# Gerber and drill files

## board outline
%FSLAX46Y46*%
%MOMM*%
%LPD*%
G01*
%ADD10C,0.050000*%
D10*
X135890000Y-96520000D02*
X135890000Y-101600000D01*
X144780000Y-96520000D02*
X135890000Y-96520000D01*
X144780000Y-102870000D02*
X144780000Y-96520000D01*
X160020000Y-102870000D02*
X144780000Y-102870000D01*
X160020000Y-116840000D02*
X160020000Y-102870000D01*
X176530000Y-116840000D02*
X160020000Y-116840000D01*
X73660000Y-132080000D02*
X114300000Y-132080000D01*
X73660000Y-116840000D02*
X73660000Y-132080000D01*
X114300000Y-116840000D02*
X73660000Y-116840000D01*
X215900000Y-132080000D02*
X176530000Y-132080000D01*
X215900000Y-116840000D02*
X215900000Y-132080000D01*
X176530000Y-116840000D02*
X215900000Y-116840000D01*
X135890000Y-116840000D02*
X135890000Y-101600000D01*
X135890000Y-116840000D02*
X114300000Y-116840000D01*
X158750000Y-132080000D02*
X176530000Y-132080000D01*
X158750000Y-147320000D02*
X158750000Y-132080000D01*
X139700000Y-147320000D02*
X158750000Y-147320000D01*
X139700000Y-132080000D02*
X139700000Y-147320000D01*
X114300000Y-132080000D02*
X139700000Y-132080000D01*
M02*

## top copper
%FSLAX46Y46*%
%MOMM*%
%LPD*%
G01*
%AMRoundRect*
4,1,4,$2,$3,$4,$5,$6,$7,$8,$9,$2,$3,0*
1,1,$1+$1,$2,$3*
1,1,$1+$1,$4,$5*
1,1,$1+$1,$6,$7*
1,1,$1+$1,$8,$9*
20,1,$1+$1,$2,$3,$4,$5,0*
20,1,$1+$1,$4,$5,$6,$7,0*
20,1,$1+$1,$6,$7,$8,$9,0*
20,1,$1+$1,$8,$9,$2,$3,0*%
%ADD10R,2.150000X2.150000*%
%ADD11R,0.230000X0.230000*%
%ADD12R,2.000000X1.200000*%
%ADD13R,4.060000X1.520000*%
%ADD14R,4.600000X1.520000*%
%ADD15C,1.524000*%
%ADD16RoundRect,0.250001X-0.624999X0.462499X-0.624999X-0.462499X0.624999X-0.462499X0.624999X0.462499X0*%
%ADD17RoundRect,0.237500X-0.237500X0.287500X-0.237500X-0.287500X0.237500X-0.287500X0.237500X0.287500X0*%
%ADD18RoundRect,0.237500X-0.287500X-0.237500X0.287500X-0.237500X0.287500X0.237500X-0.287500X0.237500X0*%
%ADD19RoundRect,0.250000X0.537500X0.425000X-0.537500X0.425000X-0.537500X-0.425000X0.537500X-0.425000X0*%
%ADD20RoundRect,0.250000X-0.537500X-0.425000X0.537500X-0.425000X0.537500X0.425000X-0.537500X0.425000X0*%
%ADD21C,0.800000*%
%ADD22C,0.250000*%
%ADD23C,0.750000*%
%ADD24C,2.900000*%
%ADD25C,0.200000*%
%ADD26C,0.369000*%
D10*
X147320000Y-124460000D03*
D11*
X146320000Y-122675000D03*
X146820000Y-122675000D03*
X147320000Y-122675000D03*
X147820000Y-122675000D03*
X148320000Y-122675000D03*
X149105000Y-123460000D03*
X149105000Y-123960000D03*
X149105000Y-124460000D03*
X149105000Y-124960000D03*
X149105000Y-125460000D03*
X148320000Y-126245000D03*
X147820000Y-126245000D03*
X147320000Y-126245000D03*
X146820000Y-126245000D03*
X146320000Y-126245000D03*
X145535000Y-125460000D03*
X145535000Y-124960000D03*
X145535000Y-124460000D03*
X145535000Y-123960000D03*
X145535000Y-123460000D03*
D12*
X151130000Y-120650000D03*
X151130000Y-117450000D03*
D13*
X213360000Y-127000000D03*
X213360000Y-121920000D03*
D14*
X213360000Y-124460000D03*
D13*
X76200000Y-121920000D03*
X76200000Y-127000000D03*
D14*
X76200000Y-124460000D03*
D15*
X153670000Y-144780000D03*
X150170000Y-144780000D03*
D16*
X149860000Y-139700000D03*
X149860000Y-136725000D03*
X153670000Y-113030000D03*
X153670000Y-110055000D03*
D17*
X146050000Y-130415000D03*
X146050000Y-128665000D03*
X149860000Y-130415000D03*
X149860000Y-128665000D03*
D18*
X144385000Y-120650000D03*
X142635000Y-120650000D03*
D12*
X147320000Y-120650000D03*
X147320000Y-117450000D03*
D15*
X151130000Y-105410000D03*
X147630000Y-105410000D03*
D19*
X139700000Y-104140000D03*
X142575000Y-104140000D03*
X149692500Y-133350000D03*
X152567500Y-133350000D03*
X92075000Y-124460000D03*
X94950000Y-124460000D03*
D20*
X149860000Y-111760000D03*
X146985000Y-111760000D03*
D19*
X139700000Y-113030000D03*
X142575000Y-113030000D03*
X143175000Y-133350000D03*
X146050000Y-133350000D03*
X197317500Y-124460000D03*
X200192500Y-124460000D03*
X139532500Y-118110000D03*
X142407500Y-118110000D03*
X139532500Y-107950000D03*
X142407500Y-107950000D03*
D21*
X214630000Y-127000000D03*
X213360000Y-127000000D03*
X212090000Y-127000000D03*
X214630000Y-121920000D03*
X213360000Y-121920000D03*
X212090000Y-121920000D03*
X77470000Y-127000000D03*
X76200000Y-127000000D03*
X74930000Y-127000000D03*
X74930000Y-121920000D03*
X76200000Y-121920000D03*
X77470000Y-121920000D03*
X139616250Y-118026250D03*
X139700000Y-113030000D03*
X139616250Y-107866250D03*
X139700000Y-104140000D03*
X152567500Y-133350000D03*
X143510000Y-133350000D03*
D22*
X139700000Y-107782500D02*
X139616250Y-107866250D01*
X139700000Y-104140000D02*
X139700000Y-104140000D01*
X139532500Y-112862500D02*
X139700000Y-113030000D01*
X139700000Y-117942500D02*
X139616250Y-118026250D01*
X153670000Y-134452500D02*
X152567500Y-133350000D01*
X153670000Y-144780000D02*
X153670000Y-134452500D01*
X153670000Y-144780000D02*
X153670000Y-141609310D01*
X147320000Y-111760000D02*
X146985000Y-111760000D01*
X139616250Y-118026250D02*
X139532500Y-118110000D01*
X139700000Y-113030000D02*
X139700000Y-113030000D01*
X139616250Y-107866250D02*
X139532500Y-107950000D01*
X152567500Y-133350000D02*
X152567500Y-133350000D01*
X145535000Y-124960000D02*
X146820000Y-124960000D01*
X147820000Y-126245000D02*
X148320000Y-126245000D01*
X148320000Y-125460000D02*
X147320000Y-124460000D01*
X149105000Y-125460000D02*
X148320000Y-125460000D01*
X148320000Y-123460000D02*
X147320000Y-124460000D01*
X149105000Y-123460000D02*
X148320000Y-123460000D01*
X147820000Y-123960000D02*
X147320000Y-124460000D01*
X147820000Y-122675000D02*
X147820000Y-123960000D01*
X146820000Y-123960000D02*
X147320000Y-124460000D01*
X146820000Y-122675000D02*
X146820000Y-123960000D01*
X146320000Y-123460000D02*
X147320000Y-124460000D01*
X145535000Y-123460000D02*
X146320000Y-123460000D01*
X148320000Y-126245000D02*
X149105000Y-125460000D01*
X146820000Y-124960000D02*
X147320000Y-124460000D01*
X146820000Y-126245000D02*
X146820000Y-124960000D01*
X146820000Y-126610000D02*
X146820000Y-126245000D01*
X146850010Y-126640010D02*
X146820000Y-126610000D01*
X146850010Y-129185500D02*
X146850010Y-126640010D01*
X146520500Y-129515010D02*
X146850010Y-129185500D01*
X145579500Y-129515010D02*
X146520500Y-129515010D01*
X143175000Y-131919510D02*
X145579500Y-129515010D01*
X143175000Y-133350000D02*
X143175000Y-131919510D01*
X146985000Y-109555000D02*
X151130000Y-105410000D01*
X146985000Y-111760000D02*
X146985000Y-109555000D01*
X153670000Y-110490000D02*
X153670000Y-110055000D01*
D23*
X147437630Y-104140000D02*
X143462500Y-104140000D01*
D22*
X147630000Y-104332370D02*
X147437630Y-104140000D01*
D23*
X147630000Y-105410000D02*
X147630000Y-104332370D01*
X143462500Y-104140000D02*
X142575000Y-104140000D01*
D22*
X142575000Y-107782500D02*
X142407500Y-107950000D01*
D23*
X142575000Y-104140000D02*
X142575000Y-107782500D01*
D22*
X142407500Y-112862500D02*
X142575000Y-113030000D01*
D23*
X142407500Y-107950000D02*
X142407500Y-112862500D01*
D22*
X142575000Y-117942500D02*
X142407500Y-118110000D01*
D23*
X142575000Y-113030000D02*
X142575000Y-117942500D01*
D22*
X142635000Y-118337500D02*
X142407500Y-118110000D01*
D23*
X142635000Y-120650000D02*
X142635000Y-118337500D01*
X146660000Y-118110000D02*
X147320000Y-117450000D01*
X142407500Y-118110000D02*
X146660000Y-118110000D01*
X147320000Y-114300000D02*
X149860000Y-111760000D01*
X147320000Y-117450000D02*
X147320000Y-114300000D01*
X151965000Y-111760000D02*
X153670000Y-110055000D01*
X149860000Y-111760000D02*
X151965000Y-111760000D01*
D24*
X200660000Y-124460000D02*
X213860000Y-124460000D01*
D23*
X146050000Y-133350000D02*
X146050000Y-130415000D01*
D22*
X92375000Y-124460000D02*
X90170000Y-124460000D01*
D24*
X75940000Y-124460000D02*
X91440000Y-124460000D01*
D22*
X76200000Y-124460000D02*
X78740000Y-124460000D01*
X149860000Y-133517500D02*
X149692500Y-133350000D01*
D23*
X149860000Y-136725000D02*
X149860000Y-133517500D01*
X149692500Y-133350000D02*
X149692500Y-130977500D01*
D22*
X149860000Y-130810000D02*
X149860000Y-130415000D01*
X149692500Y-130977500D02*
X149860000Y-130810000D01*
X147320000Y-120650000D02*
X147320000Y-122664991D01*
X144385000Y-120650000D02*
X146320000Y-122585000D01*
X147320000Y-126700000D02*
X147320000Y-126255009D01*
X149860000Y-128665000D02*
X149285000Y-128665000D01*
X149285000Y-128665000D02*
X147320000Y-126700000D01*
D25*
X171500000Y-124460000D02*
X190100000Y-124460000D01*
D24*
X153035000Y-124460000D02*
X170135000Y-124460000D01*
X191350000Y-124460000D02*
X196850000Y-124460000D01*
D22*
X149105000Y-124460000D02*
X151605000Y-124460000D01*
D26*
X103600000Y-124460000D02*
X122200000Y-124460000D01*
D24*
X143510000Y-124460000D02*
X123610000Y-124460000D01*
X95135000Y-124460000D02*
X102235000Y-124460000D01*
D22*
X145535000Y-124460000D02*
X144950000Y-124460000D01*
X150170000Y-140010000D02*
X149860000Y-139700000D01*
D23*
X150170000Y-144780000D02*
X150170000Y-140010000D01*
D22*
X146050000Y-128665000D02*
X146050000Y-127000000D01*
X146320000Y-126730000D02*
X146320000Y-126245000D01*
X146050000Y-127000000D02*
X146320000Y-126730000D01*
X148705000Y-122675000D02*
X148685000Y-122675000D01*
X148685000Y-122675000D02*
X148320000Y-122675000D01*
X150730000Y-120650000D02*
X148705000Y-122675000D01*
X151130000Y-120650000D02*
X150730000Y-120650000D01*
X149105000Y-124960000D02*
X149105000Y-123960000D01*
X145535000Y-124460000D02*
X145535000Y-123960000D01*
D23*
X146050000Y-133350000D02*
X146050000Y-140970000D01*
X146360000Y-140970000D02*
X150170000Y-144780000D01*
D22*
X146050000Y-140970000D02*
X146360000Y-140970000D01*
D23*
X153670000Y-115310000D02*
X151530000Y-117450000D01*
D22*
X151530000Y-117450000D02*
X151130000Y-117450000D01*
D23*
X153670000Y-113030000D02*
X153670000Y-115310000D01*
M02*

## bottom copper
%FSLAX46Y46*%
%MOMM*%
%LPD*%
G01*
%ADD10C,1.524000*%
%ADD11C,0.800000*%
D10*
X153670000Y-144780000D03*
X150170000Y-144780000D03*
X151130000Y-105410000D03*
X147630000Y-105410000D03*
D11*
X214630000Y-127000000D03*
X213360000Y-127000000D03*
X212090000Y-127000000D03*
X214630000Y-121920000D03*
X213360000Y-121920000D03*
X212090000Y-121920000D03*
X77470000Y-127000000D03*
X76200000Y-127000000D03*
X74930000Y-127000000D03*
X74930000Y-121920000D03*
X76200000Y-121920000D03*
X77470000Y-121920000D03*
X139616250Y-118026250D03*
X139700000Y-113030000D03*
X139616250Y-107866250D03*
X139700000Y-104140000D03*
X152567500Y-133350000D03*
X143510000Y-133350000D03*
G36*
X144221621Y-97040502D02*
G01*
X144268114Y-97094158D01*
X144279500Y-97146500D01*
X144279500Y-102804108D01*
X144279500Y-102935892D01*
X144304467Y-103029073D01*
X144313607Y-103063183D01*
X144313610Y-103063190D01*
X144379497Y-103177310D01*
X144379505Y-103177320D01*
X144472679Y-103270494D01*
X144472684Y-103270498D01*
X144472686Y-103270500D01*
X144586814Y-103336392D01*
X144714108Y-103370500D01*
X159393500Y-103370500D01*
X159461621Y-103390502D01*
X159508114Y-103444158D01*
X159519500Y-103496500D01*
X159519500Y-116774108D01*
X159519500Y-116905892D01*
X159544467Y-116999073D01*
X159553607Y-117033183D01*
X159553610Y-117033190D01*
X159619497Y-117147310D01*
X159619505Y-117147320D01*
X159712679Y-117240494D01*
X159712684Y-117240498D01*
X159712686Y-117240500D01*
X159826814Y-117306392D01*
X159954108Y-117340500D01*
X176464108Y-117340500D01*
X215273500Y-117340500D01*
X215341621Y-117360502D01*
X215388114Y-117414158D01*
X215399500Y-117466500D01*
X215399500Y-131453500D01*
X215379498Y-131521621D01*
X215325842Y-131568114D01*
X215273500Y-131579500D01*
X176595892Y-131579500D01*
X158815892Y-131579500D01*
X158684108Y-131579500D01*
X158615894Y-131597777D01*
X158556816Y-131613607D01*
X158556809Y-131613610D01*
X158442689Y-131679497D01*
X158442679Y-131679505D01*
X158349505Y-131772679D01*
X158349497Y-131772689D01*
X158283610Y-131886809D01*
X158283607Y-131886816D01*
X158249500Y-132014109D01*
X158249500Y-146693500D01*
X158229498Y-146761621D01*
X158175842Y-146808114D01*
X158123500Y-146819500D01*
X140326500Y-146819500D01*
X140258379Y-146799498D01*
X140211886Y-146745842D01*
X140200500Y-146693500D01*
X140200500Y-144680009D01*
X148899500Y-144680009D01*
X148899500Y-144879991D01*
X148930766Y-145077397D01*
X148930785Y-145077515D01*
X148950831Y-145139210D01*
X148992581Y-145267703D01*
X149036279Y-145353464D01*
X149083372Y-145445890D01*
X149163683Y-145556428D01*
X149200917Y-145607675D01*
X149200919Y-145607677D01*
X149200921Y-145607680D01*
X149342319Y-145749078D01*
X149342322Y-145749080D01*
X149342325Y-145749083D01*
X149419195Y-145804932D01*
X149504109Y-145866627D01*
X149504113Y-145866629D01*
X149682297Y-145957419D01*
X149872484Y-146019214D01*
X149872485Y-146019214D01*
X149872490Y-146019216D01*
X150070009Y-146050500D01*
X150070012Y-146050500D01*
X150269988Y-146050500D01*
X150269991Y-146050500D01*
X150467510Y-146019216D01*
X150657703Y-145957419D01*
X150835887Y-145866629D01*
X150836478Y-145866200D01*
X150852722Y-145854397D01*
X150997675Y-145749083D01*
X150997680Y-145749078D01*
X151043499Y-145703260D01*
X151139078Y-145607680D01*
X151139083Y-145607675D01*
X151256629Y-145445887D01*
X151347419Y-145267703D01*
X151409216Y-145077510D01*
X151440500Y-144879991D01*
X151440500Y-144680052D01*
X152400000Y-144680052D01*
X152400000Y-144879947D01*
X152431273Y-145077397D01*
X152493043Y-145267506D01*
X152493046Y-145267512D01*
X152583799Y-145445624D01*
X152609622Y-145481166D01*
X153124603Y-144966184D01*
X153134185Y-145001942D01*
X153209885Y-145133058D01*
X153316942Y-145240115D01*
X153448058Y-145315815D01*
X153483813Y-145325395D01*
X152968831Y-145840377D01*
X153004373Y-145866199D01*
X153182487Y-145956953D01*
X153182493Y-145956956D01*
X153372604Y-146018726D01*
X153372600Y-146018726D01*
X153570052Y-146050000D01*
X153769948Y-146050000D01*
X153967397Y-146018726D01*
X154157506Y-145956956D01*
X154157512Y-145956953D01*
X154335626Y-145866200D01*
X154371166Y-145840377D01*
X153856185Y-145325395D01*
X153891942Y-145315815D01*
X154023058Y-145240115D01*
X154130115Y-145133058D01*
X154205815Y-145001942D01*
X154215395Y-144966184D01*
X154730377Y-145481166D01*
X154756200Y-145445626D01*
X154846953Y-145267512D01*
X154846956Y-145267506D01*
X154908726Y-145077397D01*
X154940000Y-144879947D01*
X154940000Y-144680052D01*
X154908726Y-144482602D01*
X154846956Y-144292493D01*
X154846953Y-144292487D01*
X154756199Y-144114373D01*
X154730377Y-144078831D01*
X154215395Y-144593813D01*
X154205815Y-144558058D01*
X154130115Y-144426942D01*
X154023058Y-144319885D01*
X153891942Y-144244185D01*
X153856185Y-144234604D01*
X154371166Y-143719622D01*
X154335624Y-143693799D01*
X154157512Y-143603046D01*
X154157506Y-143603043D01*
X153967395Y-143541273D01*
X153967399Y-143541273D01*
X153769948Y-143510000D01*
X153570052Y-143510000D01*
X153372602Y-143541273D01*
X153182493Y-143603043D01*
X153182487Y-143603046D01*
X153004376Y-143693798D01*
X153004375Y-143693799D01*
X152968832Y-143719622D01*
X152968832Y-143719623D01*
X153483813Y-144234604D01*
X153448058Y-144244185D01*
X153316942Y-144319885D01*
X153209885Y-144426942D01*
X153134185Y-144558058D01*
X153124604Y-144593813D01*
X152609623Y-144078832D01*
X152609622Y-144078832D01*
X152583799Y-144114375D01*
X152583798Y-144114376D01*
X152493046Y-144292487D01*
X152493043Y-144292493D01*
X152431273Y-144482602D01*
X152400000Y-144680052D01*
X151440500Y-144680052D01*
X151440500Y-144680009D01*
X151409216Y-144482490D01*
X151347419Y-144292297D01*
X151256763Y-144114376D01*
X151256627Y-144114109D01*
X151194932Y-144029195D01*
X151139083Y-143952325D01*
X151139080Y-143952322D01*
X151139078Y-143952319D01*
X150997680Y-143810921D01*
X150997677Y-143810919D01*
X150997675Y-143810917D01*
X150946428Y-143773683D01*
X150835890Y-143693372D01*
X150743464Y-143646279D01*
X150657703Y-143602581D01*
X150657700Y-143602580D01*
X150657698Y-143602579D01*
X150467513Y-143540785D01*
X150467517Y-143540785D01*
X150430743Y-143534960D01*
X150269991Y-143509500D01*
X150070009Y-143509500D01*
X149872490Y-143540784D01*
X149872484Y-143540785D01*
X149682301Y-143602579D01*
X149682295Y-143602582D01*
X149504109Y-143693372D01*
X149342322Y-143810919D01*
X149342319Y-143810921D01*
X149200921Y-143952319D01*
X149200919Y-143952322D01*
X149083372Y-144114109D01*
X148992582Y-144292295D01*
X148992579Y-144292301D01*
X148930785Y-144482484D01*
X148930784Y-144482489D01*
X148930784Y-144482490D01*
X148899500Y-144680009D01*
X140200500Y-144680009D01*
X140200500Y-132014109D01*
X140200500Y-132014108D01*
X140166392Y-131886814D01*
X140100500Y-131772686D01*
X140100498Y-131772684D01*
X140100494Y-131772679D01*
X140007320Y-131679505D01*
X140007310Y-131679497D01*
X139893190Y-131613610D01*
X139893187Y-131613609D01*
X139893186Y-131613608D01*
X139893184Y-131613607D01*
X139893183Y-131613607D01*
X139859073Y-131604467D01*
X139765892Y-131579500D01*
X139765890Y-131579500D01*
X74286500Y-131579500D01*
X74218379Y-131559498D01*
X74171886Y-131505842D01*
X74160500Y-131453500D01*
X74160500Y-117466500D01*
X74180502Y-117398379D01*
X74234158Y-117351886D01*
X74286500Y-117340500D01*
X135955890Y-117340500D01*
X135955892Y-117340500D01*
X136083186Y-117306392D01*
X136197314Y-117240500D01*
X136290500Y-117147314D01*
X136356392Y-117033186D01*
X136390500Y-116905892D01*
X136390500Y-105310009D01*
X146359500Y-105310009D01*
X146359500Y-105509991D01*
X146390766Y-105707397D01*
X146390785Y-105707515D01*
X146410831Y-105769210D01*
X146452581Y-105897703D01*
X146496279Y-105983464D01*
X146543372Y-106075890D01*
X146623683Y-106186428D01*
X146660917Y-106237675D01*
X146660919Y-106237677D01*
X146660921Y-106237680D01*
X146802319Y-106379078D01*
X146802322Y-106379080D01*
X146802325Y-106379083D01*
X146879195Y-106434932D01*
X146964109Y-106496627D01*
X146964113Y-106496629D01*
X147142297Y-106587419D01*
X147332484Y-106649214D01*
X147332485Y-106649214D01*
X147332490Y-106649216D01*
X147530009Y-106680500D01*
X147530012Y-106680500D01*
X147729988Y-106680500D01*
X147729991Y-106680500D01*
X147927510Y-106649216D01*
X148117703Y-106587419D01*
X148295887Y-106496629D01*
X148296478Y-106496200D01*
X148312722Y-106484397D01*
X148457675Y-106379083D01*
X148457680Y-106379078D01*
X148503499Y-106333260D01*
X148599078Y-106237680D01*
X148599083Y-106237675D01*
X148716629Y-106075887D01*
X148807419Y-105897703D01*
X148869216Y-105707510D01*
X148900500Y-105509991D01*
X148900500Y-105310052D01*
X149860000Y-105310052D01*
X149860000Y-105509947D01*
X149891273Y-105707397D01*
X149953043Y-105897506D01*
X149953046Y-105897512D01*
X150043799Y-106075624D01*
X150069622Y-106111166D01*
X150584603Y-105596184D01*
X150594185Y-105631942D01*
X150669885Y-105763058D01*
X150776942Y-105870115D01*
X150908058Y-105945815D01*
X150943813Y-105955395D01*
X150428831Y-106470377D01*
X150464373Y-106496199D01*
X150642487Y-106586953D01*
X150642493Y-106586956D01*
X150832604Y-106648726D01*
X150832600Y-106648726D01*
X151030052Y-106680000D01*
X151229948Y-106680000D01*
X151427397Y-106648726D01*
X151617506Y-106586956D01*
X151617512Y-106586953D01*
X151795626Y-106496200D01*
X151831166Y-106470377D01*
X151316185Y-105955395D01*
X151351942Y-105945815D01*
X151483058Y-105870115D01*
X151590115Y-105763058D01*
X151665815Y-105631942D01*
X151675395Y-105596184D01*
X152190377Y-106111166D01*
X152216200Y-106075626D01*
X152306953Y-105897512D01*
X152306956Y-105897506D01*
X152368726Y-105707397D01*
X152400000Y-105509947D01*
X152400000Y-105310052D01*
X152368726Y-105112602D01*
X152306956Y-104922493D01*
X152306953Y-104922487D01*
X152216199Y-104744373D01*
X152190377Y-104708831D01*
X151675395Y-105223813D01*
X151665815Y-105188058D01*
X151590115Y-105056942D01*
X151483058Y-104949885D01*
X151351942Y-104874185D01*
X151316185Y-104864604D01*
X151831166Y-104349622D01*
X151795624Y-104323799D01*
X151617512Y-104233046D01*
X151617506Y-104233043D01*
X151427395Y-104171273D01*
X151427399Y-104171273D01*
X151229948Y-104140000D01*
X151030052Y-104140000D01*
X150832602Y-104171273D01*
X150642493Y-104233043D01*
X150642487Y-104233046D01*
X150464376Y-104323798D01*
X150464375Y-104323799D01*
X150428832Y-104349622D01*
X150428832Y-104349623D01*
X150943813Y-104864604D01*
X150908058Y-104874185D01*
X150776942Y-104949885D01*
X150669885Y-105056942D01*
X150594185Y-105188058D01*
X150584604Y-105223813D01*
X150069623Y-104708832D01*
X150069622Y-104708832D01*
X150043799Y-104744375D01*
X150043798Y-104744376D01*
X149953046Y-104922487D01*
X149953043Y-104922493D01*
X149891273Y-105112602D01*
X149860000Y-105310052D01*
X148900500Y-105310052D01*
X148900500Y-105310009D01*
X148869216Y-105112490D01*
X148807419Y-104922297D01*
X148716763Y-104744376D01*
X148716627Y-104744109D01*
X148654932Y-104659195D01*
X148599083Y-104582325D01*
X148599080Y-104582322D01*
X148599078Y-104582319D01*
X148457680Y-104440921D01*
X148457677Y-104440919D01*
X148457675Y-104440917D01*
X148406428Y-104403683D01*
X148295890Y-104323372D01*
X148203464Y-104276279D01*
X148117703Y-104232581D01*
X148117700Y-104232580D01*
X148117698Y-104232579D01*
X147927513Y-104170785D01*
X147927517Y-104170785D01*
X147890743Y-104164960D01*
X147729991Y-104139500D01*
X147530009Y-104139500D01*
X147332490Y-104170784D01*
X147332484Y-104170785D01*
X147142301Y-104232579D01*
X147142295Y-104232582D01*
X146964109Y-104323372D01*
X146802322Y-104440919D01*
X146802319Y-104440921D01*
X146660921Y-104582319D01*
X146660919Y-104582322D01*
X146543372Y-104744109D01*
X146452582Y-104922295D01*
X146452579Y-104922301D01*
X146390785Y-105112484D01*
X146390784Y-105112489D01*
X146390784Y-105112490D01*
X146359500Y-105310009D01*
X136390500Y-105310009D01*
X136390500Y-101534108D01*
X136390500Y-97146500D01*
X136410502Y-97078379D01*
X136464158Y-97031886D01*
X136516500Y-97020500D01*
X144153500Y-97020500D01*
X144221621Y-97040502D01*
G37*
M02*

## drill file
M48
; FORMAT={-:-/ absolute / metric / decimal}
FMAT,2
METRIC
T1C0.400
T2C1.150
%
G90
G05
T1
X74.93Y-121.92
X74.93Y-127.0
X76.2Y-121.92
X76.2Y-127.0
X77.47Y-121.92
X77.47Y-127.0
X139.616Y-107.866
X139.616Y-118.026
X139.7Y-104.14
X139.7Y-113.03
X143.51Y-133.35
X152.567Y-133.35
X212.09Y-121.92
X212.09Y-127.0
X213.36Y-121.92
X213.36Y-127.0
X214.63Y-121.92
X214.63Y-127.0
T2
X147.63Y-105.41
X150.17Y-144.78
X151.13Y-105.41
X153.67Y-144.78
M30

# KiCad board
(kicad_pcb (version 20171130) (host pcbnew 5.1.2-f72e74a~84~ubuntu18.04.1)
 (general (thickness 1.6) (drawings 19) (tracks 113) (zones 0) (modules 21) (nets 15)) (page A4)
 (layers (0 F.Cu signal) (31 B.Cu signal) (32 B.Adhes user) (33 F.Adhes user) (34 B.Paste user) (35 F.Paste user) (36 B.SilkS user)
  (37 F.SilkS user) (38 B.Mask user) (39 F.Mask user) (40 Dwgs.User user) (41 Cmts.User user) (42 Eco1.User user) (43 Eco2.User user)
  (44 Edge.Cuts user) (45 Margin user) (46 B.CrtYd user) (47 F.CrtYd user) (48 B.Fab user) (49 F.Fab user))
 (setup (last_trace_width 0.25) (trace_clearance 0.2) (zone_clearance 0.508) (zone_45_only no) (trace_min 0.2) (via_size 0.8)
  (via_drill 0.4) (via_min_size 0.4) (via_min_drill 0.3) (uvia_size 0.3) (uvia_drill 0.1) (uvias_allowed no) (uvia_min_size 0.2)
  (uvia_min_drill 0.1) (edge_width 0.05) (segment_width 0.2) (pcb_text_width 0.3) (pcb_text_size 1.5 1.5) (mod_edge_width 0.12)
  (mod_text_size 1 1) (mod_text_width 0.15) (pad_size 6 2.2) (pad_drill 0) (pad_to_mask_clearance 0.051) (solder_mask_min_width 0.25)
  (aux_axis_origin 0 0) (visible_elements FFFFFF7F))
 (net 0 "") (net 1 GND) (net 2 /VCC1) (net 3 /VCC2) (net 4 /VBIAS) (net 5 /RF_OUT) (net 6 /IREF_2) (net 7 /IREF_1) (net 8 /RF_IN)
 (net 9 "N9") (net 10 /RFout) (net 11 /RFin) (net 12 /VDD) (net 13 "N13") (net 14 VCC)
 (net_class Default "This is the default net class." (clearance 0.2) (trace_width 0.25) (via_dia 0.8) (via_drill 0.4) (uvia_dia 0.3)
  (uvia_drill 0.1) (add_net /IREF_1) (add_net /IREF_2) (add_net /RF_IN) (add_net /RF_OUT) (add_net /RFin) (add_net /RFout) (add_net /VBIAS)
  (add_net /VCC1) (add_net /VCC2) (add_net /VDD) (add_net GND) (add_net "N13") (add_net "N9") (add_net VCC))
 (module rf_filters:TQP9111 (layer F.Cu) (at 147.32 124.46)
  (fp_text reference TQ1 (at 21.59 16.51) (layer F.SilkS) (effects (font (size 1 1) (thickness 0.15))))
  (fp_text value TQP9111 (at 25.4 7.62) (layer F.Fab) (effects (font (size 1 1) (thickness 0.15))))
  (pad 21 smd rect (at 0 0) (size 2.15 2.15) (layers F.Cu F.Paste F.Mask) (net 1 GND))
  (pad 20 smd rect (at -1 -1.785) (size 0.23 0.23) (layers F.Cu F.Paste F.Mask) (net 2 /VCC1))
  (pad 19 smd rect (at -0.5 -1.785) (size 0.23 0.23) (layers F.Cu F.Paste F.Mask) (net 1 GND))
  (pad 18 smd rect (at 0 -1.785) (size 0.23 0.23) (layers F.Cu F.Paste F.Mask) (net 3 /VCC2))
  (pad 17 smd rect (at 0.5 -1.785) (size 0.23 0.23) (layers F.Cu F.Paste F.Mask) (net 1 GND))
  (pad 16 smd rect (at 1 -1.785) (size 0.23 0.23) (layers F.Cu F.Paste F.Mask) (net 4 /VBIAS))
  (pad 15 smd rect (at 1.785 -1) (size 0.23 0.23) (layers F.Cu F.Paste F.Mask) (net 1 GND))
  (pad 14 smd rect (at 1.785 -0.5) (size 0.23 0.23) (layers F.Cu F.Paste F.Mask) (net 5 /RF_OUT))
  (pad 13 smd rect (at 1.785 0) (size 0.23 0.23) (layers F.Cu F.Paste F.Mask) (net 5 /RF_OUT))
  (pad 12 smd rect (at 1.785 0.5) (size 0.23 0.23) (layers F.Cu F.Paste F.Mask) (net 5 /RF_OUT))
  (pad 11 smd rect (at 1.785 1) (size 0.23 0.23) (layers F.Cu F.Paste F.Mask) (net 1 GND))
  (pad 10 smd rect (at 1 1.785) (size 0.23 0.23) (layers F.Cu F.Paste F.Mask) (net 1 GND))
  (pad 9 smd rect (at 0.5 1.785) (size 0.23 0.23) (layers F.Cu F.Paste F.Mask) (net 1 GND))
  (pad 8 smd rect (at 0 1.785) (size 0.23 0.23) (layers F.Cu F.Paste F.Mask) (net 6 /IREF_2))
  (pad 7 smd rect (at -0.5 1.785) (size 0.23 0.23) (layers F.Cu F.Paste F.Mask) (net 1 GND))
  (pad 6 smd rect (at -1 1.785) (size 0.23 0.23) (layers F.Cu F.Paste F.Mask) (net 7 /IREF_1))
  (pad 5 smd rect (at -1.785 1) (size 0.23 0.23) (layers F.Cu F.Paste F.Mask))
  (pad 4 smd rect (at -1.785 0.5) (size 0.23 0.23) (layers F.Cu F.Paste F.Mask) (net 1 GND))
  (pad 3 smd rect (at -1.785 0) (size 0.23 0.23) (layers F.Cu F.Paste F.Mask) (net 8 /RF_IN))
  (pad 2 smd rect (at -1.785 -0.5) (size 0.23 0.23) (layers F.Cu F.Paste F.Mask) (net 8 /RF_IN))
  (pad 1 smd rect (at -1.785 -1) (size 0.23 0.23) (layers F.Cu F.Paste F.Mask) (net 1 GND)))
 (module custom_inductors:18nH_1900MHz (layer F.Cu) (at 151.13 119.05)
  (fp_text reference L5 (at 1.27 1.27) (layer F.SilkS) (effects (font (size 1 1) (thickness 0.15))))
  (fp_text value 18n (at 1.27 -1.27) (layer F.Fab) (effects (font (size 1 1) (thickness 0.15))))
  (pad 2 smd rect (at 0 1.6) (size 2 1.2) (layers F.Cu F.Paste F.Mask) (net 4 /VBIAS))
  (pad 1 smd rect (at 0 -1.6) (size 2 1.2) (layers F.Cu F.Paste F.Mask) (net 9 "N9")))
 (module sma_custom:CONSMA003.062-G (layer F.Cu) (at 217.17 127)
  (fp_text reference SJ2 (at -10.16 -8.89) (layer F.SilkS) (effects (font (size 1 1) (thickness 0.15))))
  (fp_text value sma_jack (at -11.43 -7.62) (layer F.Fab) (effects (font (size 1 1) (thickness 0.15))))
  (pad 3 smd rect (at -3.81 0) (size 4.06 1.52) (layers F.Cu F.Paste F.Mask) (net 1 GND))
  (pad 2 smd rect (at -3.81 -5.08) (size 4.06 1.52) (layers F.Cu F.Paste F.Mask) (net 1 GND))
  (pad 1 smd rect (at -3.81 -2.54) (size 4.6 1.52) (layers F.Cu F.Paste F.Mask) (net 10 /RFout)))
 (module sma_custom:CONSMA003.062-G (layer F.Cu) (at 72.39 121.92 180)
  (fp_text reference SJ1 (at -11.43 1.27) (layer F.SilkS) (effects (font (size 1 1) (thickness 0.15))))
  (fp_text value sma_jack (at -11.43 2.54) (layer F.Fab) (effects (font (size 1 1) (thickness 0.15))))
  (pad 3 smd rect (at -3.81 0 180) (size 4.06 1.52) (layers F.Cu F.Paste F.Mask) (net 1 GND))
  (pad 2 smd rect (at -3.81 -5.08 180) (size 4.06 1.52) (layers F.Cu F.Paste F.Mask) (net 1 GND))
  (pad 1 smd rect (at -3.81 -2.54 180) (size 4.6 1.52) (layers F.Cu F.Paste F.Mask) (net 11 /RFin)))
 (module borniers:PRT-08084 (layer F.Cu) (at 153.67 149.86)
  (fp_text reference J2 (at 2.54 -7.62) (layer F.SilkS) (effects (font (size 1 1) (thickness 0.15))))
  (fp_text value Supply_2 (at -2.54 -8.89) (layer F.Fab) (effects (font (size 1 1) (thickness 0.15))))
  (pad 2 thru_hole circle (at 0 -5.08) (size 1.524 1.524) (drill 1.15) (layers *.Cu *.Mask) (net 1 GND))
  (pad 1 thru_hole circle (at -3.5 -5.08) (size 1.524 1.524) (drill 1.15) (layers *.Cu *.Mask) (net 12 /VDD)))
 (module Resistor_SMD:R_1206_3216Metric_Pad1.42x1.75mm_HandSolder (layer F.Cu) (at 149.86 138.2125 270)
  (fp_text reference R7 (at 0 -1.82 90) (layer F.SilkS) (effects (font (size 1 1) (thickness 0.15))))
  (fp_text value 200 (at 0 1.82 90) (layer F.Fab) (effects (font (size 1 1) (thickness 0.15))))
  (pad 2 smd roundrect (at 1.4875 0 270) (size 1.425 1.75) (layers F.Cu F.Paste F.Mask) (roundrect_rratio 0.175439) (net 12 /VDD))
  (pad 1 smd roundrect (at -1.4875 0 270) (size 1.425 1.75) (layers F.Cu F.Paste F.Mask) (roundrect_rratio 0.175439) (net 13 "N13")))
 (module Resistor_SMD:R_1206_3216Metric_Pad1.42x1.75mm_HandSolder (layer F.Cu) (at 153.67 111.5425 270)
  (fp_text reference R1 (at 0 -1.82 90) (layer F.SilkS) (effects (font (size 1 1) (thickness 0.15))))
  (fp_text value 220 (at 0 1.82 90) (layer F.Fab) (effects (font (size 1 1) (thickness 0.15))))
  (pad 2 smd roundrect (at 1.4875 0 270) (size 1.425 1.75) (layers F.Cu F.Paste F.Mask) (roundrect_rratio 0.175439) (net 9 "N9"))
  (pad 1 smd roundrect (at -1.4875 0 270) (size 1.425 1.75) (layers F.Cu F.Paste F.Mask) (roundrect_rratio 0.175439) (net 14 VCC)))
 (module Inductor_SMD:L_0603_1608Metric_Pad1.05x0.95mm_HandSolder (layer F.Cu) (at 146.05 129.54 270)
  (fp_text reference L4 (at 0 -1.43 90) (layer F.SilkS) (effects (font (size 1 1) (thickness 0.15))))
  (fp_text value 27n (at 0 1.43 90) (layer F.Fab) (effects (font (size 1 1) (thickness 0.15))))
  (pad 2 smd roundrect (at 0.875 0 270) (size 1.05 0.95) (layers F.Cu F.Paste F.Mask) (roundrect_rratio 0.25) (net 12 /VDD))
  (pad 1 smd roundrect (at -0.875 0 270) (size 1.05 0.95) (layers F.Cu F.Paste F.Mask) (roundrect_rratio 0.25) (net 7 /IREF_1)))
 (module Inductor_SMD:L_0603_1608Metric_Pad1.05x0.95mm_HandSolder (layer F.Cu) (at 149.86 129.54 270)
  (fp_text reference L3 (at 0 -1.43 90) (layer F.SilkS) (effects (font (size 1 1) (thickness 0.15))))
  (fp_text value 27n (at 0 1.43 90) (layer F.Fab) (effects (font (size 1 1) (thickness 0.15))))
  (pad 2 smd roundrect (at 0.875 0 270) (size 1.05 0.95) (layers F.Cu F.Paste F.Mask) (roundrect_rratio 0.25) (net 13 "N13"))
  (pad 1 smd roundrect (at -0.875 0 270) (size 1.05 0.95) (layers F.Cu F.Paste F.Mask) (roundrect_rratio 0.25) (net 6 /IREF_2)))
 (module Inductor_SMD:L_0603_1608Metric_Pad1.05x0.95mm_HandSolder (layer F.Cu) (at 143.51 120.65)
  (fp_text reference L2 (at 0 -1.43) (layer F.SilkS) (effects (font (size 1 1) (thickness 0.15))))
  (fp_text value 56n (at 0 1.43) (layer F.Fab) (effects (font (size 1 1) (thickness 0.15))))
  (pad 2 smd roundrect (at 0.875 0) (size 1.05 0.95) (layers F.Cu F.Paste F.Mask) (roundrect_rratio 0.25) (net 2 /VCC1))
  (pad 1 smd roundrect (at -0.875 0) (size 1.05 0.95) (layers F.Cu F.Paste F.Mask) (roundrect_rratio 0.25) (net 14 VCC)))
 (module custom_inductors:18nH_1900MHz (layer F.Cu) (at 147.32 119.05)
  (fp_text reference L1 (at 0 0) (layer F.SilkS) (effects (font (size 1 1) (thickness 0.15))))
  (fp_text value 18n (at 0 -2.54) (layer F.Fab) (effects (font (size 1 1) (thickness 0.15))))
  (pad 2 smd rect (at 0 1.6) (size 2 1.2) (layers F.Cu F.Paste F.Mask) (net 3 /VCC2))
  (pad 1 smd rect (at 0 -1.6) (size 2 1.2) (layers F.Cu F.Paste F.Mask) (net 14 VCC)))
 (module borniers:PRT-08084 (layer F.Cu) (at 151.13 110.49)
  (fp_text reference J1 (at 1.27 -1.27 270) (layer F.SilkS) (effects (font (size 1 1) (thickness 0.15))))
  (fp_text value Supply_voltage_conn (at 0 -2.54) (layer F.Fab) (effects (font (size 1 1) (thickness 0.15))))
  (pad 2 thru_hole circle (at 0 -5.08) (size 1.524 1.524) (drill 1.15) (layers *.Cu *.Mask) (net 1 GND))
  (pad 1 thru_hole circle (at -3.5 -5.08) (size 1.524 1.524) (drill 1.15) (layers *.Cu *.Mask) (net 14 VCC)))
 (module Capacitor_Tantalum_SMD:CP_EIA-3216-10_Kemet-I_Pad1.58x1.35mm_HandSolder (layer F.Cu) (at 141.1375 104.14 180)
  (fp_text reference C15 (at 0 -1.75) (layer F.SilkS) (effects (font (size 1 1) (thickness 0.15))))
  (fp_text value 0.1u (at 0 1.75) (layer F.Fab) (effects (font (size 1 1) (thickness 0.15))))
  (pad 2 smd roundrect (at 1.4375 0 180) (size 1.575 1.35) (layers F.Cu F.Paste F.Mask) (roundrect_rratio 0.185185) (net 1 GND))
  (pad 1 smd roundrect (at -1.4375 0 180) (size 1.575 1.35) (layers F.Cu F.Paste F.Mask) (roundrect_rratio 0.185185) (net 14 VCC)))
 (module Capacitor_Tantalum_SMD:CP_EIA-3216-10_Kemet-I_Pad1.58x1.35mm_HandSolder (layer F.Cu) (at 151.13 133.35 180)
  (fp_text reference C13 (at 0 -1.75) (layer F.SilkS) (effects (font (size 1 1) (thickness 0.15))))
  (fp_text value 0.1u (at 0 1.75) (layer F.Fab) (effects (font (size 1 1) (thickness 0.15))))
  (pad 2 smd roundrect (at 1.4375 0 180) (size 1.575 1.35) (layers F.Cu F.Paste F.Mask) (roundrect_rratio 0.185185) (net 13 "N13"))
  (pad 1 smd roundrect (at -1.4375 0 180) (size 1.575 1.35) (layers F.Cu F.Paste F.Mask) (roundrect_rratio 0.185185) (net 1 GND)))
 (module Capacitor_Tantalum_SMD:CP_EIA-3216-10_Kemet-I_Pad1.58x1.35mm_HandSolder (layer F.Cu) (at 93.5125 124.46 180)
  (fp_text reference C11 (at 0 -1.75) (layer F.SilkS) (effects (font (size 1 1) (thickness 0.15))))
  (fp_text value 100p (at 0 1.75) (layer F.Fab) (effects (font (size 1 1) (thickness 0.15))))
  (pad 2 smd roundrect (at 1.4375 0 180) (size 1.575 1.35) (layers F.Cu F.Paste F.Mask) (roundrect_rratio 0.185185) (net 11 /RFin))
  (pad 1 smd roundrect (at -1.4375 0 180) (size 1.575 1.35) (layers F.Cu F.Paste F.Mask) (roundrect_rratio 0.185185) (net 8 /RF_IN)))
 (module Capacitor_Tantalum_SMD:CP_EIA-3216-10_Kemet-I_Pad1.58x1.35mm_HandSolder (layer F.Cu) (at 148.4225 111.76)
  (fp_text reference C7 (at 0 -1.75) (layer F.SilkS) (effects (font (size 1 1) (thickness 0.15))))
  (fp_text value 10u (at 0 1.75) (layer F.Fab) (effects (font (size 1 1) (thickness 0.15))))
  (pad 2 smd roundrect (at 1.4375 0) (size 1.575 1.35) (layers F.Cu F.Paste F.Mask) (roundrect_rratio 0.185185) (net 14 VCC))
  (pad 1 smd roundrect (at -1.4375 0) (size 1.575 1.35) (layers F.Cu F.Paste F.Mask) (roundrect_rratio 0.185185) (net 1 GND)))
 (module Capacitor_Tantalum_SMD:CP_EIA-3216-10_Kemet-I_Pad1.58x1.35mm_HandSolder (layer F.Cu) (at 141.1375 113.03 180)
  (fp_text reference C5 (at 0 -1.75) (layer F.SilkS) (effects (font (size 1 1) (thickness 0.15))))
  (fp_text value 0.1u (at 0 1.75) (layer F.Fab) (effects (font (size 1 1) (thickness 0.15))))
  (pad 2 smd roundrect (at 1.4375 0 180) (size 1.575 1.35) (layers F.Cu F.Paste F.Mask) (roundrect_rratio 0.185185) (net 1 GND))
  (pad 1 smd roundrect (at -1.4375 0 180) (size 1.575 1.35) (layers F.Cu F.Paste F.Mask) (roundrect_rratio 0.185185) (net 14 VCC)))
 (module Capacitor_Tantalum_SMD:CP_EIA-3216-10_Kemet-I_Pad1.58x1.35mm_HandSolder (layer F.Cu) (at 144.6125 133.35 180)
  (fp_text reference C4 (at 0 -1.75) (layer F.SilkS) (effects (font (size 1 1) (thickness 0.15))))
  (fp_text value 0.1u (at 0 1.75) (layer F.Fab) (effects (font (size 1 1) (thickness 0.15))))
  (pad 2 smd roundrect (at 1.4375 0 180) (size 1.575 1.35) (layers F.Cu F.Paste F.Mask) (roundrect_rratio 0.185185) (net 1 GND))
  (pad 1 smd roundrect (at -1.4375 0 180) (size 1.575 1.35) (layers F.Cu F.Paste F.Mask) (roundrect_rratio 0.185185) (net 12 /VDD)))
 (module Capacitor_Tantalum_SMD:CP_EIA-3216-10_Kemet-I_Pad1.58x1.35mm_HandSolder (layer F.Cu) (at 198.755 124.46 180)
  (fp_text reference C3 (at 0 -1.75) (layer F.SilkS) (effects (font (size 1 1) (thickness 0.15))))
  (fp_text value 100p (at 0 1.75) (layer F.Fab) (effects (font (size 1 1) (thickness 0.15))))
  (pad 2 smd roundrect (at 1.4375 0 180) (size 1.575 1.35) (layers F.Cu F.Paste F.Mask) (roundrect_rratio 0.185185) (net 5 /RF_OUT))
  (pad 1 smd roundrect (at -1.4375 0 180) (size 1.575 1.35) (layers F.Cu F.Paste F.Mask) (roundrect_rratio 0.185185) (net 10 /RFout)))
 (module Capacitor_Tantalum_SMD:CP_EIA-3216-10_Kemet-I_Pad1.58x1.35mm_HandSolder (layer F.Cu) (at 140.97 118.11 180)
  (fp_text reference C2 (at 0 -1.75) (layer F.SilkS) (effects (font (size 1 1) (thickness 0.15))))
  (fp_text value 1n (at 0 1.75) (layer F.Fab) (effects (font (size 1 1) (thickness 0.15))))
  (pad 2 smd roundrect (at 1.4375 0 180) (size 1.575 1.35) (layers F.Cu F.Paste F.Mask) (roundrect_rratio 0.185185) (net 1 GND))
  (pad 1 smd roundrect (at -1.4375 0 180) (size 1.575 1.35) (layers F.Cu F.Paste F.Mask) (roundrect_rratio 0.185185) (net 14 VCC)))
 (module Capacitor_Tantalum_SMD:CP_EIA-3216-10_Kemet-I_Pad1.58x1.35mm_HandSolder (layer F.Cu) (at 140.97 107.95 180)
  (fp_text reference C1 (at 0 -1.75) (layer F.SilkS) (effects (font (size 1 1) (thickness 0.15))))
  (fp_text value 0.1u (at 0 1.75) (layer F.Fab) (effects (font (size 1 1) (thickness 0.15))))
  (pad 2 smd roundrect (at 1.4375 0 180) (size 1.575 1.35) (layers F.Cu F.Paste F.Mask) (roundrect_rratio 0.185185) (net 1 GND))
  (pad 1 smd roundrect (at -1.4375 0 180) (size 1.575 1.35) (layers F.Cu F.Paste F.Mask) (roundrect_rratio 0.185185) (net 14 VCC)))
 (gr_line (start 135.89 96.52) (end 135.89 101.6) (layer Edge.Cuts) (width 0.05))
 (gr_line (start 144.78 96.52) (end 135.89 96.52) (layer Edge.Cuts) (width 0.05))
 (gr_line (start 144.78 102.87) (end 144.78 96.52) (layer Edge.Cuts) (width 0.05))
 (gr_line (start 160.02 102.87) (end 144.78 102.87) (layer Edge.Cuts) (width 0.05))
 (gr_line (start 160.02 116.84) (end 160.02 102.87) (layer Edge.Cuts) (width 0.05))
 (gr_line (start 176.53 116.84) (end 160.02 116.84) (layer Edge.Cuts) (width 0.05))
 (gr_line (start 73.66 132.08) (end 114.3 132.08) (layer Edge.Cuts) (width 0.05))
 (gr_line (start 73.66 116.84) (end 73.66 132.08) (layer Edge.Cuts) (width 0.05))
 (gr_line (start 114.3 116.84) (end 73.66 116.84) (layer Edge.Cuts) (width 0.05))
 (gr_line (start 215.9 132.08) (end 176.53 132.08) (layer Edge.Cuts) (width 0.05))
 (gr_line (start 215.9 116.84) (end 215.9 132.08) (layer Edge.Cuts) (width 0.05))
 (gr_line (start 176.53 116.84) (end 215.9 116.84) (layer Edge.Cuts) (width 0.05))
 (gr_line (start 135.89 116.84) (end 135.89 101.6) (layer Edge.Cuts) (width 0.05))
 (gr_line (start 135.89 116.84) (end 114.3 116.84) (layer Edge.Cuts) (width 0.05))
 (gr_line (start 158.75 132.08) (end 176.53 132.08) (layer Edge.Cuts) (width 0.05))
 (gr_line (start 158.75 147.32) (end 158.75 132.08) (layer Edge.Cuts) (width 0.05))
 (gr_line (start 139.7 147.32) (end 158.75 147.32) (layer Edge.Cuts) (width 0.05))
 (gr_line (start 139.7 132.08) (end 139.7 147.32) (layer Edge.Cuts) (width 0.05))
 (gr_line (start 114.3 132.08) (end 139.7 132.08) (layer Edge.Cuts) (width 0.05))
 (via (at 214.63 127) (size 0.8) (drill 0.4) (layers F.Cu B.Cu) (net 1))
 (via (at 213.36 127) (size 0.8) (drill 0.4) (layers F.Cu B.Cu) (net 1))
 (via (at 212.09 127) (size 0.8) (drill 0.4) (layers F.Cu B.Cu) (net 1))
 (via (at 214.63 121.92) (size 0.8) (drill 0.4) (layers F.Cu B.Cu) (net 1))
 (via (at 213.36 121.92) (size 0.8) (drill 0.4) (layers F.Cu B.Cu) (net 1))
 (via (at 212.09 121.92) (size 0.8) (drill 0.4) (layers F.Cu B.Cu) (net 1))
 (via (at 77.47 127) (size 0.8) (drill 0.4) (layers F.Cu B.Cu) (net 1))
 (via (at 76.2 127) (size 0.8) (drill 0.4) (layers F.Cu B.Cu) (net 1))
 (via (at 74.93 127) (size 0.8) (drill 0.4) (layers F.Cu B.Cu) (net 1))
 (via (at 74.93 121.92) (size 0.8) (drill 0.4) (layers F.Cu B.Cu) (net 1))
 (via (at 76.2 121.92) (size 0.8) (drill 0.4) (layers F.Cu B.Cu) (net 1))
 (via (at 77.47 121.92) (size 0.8) (drill 0.4) (layers F.Cu B.Cu) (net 1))
 (segment (start 139.7 107.7825) (end 139.61625 107.86625) (width 0.25) (layer F.Cu) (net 1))
 (segment (start 139.7 104.14) (end 139.7 104.14) (width 0.25) (layer F.Cu) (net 1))
 (segment (start 139.5325 112.8625) (end 139.7 113.03) (width 0.25) (layer F.Cu) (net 1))
 (segment (start 139.7 117.9425) (end 139.61625 118.02625) (width 0.25) (layer F.Cu) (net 1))
 (segment (start 153.67 134.4525) (end 152.5675 133.35) (width 0.25) (layer F.Cu) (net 1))
 (segment (start 153.67 144.78) (end 153.67 134.4525) (width 0.25) (layer F.Cu) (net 1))
 (segment (start 153.67 144.78) (end 153.67 141.60931) (width 0.25) (layer F.Cu) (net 1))
 (segment (start 147.32 111.76) (end 146.985 111.76) (width 0.25) (layer F.Cu) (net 1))
 (segment (start 139.61625 118.02625) (end 139.5325 118.11) (width 0.25) (layer F.Cu) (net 1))
 (via (at 139.61625 118.02625) (size 0.8) (drill 0.4) (layers F.Cu B.Cu) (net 1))
 (segment (start 139.7 113.03) (end 139.7 113.03) (width 0.25) (layer F.Cu) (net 1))
 (via (at 139.7 113.03) (size 0.8) (drill 0.4) (layers F.Cu B.Cu) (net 1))
 (segment (start 139.61625 107.86625) (end 139.5325 107.95) (width 0.25) (layer F.Cu) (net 1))
 (via (at 139.61625 107.86625) (size 0.8) (drill 0.4) (layers F.Cu B.Cu) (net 1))
 (via (at 139.7 104.14) (size 0.8) (drill 0.4) (layers F.Cu B.Cu) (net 1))
 (segment (start 152.5675 133.35) (end 152.5675 133.35) (width 0.25) (layer F.Cu) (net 1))
 (via (at 152.5675 133.35) (size 0.8) (drill 0.4) (layers F.Cu B.Cu) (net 1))
 (segment (start 145.535 124.96) (end 146.82 124.96) (width 0.25) (layer F.Cu) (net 1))
 (segment (start 147.82 126.245) (end 148.32 126.245) (width 0.25) (layer F.Cu) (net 1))
 (segment (start 148.32 125.46) (end 147.32 124.46) (width 0.25) (layer F.Cu) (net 1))
 (segment (start 149.105 125.46) (end 148.32 125.46) (width 0.25) (layer F.Cu) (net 1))
 (segment (start 148.32 123.46) (end 147.32 124.46) (width 0.25) (layer F.Cu) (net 1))
 (segment (start 149.105 123.46) (end 148.32 123.46) (width 0.25) (layer F.Cu) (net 1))
 (segment (start 147.82 123.96) (end 147.32 124.46) (width 0.25) (layer F.Cu) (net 1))
 (segment (start 147.82 122.675) (end 147.82 123.96) (width 0.25) (layer F.Cu) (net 1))
 (segment (start 146.82 123.96) (end 147.32 124.46) (width 0.25) (layer F.Cu) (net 1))
 (segment (start 146.82 122.675) (end 146.82 123.96) (width 0.25) (layer F.Cu) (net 1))
 (segment (start 146.32 123.46) (end 147.32 124.46) (width 0.25) (layer F.Cu) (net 1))
 (segment (start 145.535 123.46) (end 146.32 123.46) (width 0.25) (layer F.Cu) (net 1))
 (segment (start 148.32 126.245) (end 149.105 125.46) (width 0.25) (layer F.Cu) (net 1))
 (segment (start 146.82 124.96) (end 147.32 124.46) (width 0.25) (layer F.Cu) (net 1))
 (segment (start 146.82 126.245) (end 146.82 124.96) (width 0.25) (layer F.Cu) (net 1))
 (segment (start 146.82 126.61) (end 146.82 126.245) (width 0.25) (layer F.Cu) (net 1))
 (segment (start 146.85001 126.64001) (end 146.82 126.61) (width 0.25) (layer F.Cu) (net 1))
 (segment (start 146.85001 129.1855) (end 146.85001 126.64001) (width 0.25) (layer F.Cu) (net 1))
 (segment (start 146.5205 129.51501) (end 146.85001 129.1855) (width 0.25) (layer F.Cu) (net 1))
 (segment (start 145.5795 129.51501) (end 146.5205 129.51501) (width 0.25) (layer F.Cu) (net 1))
 (segment (start 143.175 131.91951) (end 145.5795 129.51501) (width 0.25) (layer F.Cu) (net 1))
 (segment (start 143.175 133.35) (end 143.175 131.91951) (width 0.25) (layer F.Cu) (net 1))
 (via (at 143.51 133.35) (size 0.8) (drill 0.4) (layers F.Cu B.Cu) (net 1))
 (segment (start 146.985 109.555) (end 151.13 105.41) (width 0.25) (layer F.Cu) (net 1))
 (segment (start 146.985 111.76) (end 146.985 109.555) (width 0.25) (layer F.Cu) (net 1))
 (segment (start 153.67 110.49) (end 153.67 110.055) (width 0.25) (layer F.Cu) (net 14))
 (segment (start 147.43763 104.14) (end 143.4625 104.14) (width 0.75) (layer F.Cu) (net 14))
 (segment (start 147.63 104.33237) (end 147.43763 104.14) (width 0.25) (layer F.Cu) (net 14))
 (segment (start 147.63 105.41) (end 147.63 104.33237) (width 0.75) (layer F.Cu) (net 14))
 (segment (start 143.4625 104.14) (end 142.575 104.14) (width 0.75) (layer F.Cu) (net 14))
 (segment (start 142.575 107.7825) (end 142.4075 107.95) (width 0.25) (layer F.Cu) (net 14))
 (segment (start 142.575 104.14) (end 142.575 107.7825) (width 0.75) (layer F.Cu) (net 14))
 (segment (start 142.4075 112.8625) (end 142.575 113.03) (width 0.25) (layer F.Cu) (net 14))
 (segment (start 142.4075 107.95) (end 142.4075 112.8625) (width 0.75) (layer F.Cu) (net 14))
 (segment (start 142.575 117.9425) (end 142.4075 118.11) (width 0.25) (layer F.Cu) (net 14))
 (segment (start 142.575 113.03) (end 142.575 117.9425) (width 0.75) (layer F.Cu) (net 14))
 (segment (start 142.635 118.3375) (end 142.4075 118.11) (width 0.25) (layer F.Cu) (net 14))
 (segment (start 142.635 120.65) (end 142.635 118.3375) (width 0.75) (layer F.Cu) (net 14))
 (segment (start 146.66 118.11) (end 147.32 117.45) (width 0.75) (layer F.Cu) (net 14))
 (segment (start 142.4075 118.11) (end 146.66 118.11) (width 0.75) (layer F.Cu) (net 14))
 (segment (start 147.32 114.3) (end 149.86 111.76) (width 0.75) (layer F.Cu) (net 14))
 (segment (start 147.32 117.45) (end 147.32 114.3) (width 0.75) (layer F.Cu) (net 14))
 (segment (start 151.965 111.76) (end 153.67 110.055) (width 0.75) (layer F.Cu) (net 14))
 (segment (start 149.86 111.76) (end 151.965 111.76) (width 0.75) (layer F.Cu) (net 14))
 (segment (start 200.66 124.46) (end 213.86 124.46) (width 2.9) (layer F.Cu) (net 10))
 (segment (start 146.05 133.35) (end 146.05 130.415) (width 0.75) (layer F.Cu) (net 12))
 (segment (start 92.375 124.46) (end 90.17 124.46) (width 0.25) (layer F.Cu) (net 11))
 (segment (start 75.94 124.46) (end 91.44 124.46) (width 2.9) (layer F.Cu) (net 11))
 (segment (start 76.2 124.46) (end 78.74 124.46) (width 0.25) (layer F.Cu) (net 11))
 (segment (start 149.86 133.5175) (end 149.6925 133.35) (width 0.25) (layer F.Cu) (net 13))
 (segment (start 149.86 136.725) (end 149.86 133.5175) (width 0.75) (layer F.Cu) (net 13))
 (segment (start 149.6925 133.35) (end 149.6925 130.9775) (width 0.75) (layer F.Cu) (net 13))
 (segment (start 149.86 130.81) (end 149.86 130.415) (width 0.25) (layer F.Cu) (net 13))
 (segment (start 149.6925 130.9775) (end 149.86 130.81) (width 0.25) (layer F.Cu) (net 13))
 (segment (start 147.32 120.65) (end 147.32 122.664991) (width 0.25) (layer F.Cu) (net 3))
 (segment (start 144.385 120.65) (end 146.32 122.585) (width 0.25) (layer F.Cu) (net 2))
 (segment (start 147.32 126.7) (end 147.32 126.255009) (width 0.25) (layer F.Cu) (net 6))
 (segment (start 149.86 128.665) (end 149.285 128.665) (width 0.25) (layer F.Cu) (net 6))
 (segment (start 149.285 128.665) (end 147.32 126.7) (width 0.25) (layer F.Cu) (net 6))
 (segment (start 171.5 124.46) (end 190.1 124.46) (width 0.2) (layer F.Cu) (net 5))
 (segment (start 153.035 124.46) (end 170.135 124.46) (width 2.9) (layer F.Cu) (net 5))
 (segment (start 191.35 124.46) (end 196.85 124.46) (width 2.9) (layer F.Cu) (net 5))
 (segment (start 149.105 124.46) (end 151.605 124.46) (width 0.25) (layer F.Cu) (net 5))
 (segment (start 103.6 124.46) (end 122.2 124.46) (width 0.369) (layer F.Cu) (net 8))
 (segment (start 143.51 124.46) (end 123.61 124.46) (width 2.9) (layer F.Cu) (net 8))
 (segment (start 95.135 124.46) (end 102.235 124.46) (width 2.9) (layer F.Cu) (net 8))
 (segment (start 145.535 124.46) (end 144.95 124.46) (width 0.25) (layer F.Cu) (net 8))
 (segment (start 150.17 140.01) (end 149.86 139.7) (width 0.25) (layer F.Cu) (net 12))
 (segment (start 150.17 144.78) (end 150.17 140.01) (width 0.75) (layer F.Cu) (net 12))
 (segment (start 146.05 128.665) (end 146.05 127) (width 0.25) (layer F.Cu) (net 7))
 (segment (start 146.32 126.73) (end 146.32 126.245) (width 0.25) (layer F.Cu) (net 7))
 (segment (start 146.05 127) (end 146.32 126.73) (width 0.25) (layer F.Cu) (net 7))
 (segment (start 148.705 122.675) (end 148.685 122.675) (width 0.25) (layer F.Cu) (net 4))
 (segment (start 148.685 122.675) (end 148.32 122.675) (width 0.25) (layer F.Cu) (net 4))
 (segment (start 150.73 120.65) (end 148.705 122.675) (width 0.25) (layer F.Cu) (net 4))
 (segment (start 151.13 120.65) (end 150.73 120.65) (width 0.25) (layer F.Cu) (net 4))
 (segment (start 149.105 124.96) (end 149.105 123.96) (width 0.25) (layer F.Cu) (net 5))
 (segment (start 145.535 124.46) (end 145.535 123.96) (width 0.25) (layer F.Cu) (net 8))
 (segment (start 146.05 133.35) (end 146.05 140.97) (width 0.75) (layer F.Cu) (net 12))
 (segment (start 146.36 140.97) (end 150.17 144.78) (width 0.75) (layer F.Cu) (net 12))
 (segment (start 146.05 140.97) (end 146.36 140.97) (width 0.25) (layer F.Cu) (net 12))
 (segment (start 153.67 115.31) (end 151.53 117.45) (width 0.75) (layer F.Cu) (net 9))
 (segment (start 151.53 117.45) (end 151.13 117.45) (width 0.25) (layer F.Cu) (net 9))
 (segment (start 153.67 113.03) (end 153.67 115.31) (width 0.75) (layer F.Cu) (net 9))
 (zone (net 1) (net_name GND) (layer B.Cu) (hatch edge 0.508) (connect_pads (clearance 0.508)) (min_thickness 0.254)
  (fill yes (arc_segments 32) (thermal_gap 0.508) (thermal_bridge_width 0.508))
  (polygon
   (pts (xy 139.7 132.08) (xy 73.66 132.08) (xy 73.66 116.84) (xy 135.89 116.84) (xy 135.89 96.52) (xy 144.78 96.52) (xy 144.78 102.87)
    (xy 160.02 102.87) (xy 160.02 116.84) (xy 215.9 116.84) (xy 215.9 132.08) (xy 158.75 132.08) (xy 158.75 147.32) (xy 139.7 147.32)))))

